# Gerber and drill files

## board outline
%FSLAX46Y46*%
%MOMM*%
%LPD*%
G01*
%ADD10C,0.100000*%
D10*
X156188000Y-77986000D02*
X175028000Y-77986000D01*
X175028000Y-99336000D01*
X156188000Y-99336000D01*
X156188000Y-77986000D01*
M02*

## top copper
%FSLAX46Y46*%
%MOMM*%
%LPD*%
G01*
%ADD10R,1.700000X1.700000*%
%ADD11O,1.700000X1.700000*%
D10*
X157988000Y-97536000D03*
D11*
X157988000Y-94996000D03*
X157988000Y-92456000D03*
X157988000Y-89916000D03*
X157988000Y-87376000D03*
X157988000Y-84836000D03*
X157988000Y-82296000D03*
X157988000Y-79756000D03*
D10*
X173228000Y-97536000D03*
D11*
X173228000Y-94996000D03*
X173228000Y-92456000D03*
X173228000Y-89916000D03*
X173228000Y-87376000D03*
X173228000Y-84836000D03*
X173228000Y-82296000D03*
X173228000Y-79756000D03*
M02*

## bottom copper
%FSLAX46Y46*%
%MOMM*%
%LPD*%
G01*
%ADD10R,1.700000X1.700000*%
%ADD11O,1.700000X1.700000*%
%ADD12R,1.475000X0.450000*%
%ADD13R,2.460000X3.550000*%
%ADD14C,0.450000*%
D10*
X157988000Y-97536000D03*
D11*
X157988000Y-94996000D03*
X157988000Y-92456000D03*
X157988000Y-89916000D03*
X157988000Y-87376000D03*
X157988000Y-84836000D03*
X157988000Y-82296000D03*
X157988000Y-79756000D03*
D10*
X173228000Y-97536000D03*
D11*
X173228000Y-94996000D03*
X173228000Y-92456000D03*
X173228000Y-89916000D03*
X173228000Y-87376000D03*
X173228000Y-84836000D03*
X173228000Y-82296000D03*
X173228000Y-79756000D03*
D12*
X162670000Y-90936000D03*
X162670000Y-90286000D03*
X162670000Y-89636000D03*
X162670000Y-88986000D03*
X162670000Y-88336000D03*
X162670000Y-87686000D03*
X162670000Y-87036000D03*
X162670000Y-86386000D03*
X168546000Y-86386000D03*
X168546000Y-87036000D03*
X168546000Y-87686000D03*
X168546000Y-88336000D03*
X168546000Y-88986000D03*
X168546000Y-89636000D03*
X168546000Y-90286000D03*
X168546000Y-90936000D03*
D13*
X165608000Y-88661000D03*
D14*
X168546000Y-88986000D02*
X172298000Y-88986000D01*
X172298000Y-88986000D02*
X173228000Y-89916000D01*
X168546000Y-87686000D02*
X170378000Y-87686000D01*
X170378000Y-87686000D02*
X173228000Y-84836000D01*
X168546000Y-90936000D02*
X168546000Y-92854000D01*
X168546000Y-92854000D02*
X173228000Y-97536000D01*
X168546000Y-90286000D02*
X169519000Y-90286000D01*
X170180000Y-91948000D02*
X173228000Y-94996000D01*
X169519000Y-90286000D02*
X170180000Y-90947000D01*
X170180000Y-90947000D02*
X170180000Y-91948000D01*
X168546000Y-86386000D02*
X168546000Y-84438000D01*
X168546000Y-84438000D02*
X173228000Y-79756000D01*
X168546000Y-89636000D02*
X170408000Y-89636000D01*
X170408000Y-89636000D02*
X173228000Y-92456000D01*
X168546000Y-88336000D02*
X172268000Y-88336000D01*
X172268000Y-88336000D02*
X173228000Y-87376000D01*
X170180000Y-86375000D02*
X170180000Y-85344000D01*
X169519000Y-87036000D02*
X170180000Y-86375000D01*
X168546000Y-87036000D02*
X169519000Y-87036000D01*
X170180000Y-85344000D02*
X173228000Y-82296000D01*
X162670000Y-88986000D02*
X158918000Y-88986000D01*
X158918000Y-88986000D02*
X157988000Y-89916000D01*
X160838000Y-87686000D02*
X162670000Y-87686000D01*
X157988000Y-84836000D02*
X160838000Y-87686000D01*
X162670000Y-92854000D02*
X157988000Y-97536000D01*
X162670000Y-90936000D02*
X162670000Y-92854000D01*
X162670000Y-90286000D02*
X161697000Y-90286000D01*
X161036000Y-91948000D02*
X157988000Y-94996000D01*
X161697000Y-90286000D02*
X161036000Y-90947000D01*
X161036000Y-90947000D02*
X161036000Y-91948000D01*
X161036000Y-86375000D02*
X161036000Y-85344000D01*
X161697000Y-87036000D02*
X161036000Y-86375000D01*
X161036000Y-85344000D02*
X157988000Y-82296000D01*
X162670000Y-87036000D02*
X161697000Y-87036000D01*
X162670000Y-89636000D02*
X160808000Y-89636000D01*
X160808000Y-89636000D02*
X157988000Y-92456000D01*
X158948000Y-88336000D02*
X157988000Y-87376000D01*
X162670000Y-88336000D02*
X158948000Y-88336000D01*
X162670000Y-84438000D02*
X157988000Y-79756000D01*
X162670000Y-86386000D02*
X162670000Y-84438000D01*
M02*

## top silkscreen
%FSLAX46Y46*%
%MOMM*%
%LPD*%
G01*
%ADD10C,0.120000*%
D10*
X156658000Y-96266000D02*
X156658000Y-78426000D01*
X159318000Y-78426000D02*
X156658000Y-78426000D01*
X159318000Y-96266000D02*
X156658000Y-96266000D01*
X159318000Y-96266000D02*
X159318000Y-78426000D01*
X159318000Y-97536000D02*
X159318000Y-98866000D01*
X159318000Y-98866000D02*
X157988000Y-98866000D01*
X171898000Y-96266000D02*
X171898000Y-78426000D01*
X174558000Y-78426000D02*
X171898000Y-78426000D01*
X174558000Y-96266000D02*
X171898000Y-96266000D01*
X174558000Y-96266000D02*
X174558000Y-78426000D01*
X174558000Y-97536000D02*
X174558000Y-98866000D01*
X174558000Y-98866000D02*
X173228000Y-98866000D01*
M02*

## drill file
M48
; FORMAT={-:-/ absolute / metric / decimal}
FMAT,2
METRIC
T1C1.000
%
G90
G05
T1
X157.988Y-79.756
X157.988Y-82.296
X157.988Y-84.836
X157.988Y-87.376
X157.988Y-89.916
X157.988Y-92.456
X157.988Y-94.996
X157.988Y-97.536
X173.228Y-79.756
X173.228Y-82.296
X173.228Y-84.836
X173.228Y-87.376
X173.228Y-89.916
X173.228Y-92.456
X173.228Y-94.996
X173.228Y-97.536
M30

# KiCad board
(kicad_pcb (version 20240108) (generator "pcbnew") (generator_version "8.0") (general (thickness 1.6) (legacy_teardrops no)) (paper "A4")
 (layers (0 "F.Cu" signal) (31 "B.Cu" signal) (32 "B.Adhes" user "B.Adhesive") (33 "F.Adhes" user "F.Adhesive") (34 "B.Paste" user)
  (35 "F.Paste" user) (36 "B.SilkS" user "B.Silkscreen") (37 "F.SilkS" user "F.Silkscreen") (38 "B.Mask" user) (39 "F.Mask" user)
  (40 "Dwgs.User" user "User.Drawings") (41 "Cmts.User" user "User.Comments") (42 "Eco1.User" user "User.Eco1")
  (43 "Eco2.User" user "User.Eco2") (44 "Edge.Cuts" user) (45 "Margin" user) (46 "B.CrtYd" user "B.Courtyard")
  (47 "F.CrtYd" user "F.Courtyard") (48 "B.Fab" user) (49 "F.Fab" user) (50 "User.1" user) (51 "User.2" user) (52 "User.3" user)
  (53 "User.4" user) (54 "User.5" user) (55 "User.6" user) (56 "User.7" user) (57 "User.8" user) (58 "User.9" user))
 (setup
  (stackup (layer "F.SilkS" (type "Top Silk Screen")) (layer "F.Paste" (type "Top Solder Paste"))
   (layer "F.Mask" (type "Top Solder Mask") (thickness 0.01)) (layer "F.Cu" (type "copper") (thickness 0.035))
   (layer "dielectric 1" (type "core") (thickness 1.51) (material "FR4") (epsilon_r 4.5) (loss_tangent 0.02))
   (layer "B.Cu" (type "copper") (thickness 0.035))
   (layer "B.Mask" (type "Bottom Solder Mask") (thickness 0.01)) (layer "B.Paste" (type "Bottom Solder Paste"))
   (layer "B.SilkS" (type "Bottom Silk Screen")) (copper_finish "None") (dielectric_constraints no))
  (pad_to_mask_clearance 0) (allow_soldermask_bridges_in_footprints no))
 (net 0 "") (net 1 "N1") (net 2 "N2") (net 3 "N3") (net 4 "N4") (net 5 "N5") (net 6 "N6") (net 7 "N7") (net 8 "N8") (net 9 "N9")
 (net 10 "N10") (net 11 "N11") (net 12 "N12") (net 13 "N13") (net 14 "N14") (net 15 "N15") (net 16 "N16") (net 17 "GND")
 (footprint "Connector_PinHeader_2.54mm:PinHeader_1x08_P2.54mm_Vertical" (layer "F.Cu") (at 157.988 97.536 180)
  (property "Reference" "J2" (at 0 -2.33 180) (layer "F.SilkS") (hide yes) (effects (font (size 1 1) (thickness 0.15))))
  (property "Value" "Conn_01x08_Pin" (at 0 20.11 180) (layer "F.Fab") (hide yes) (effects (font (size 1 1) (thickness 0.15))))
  (fp_line (start 1.33 1.27) (end 1.33 19.11) (stroke (width 0.12) (type solid)) (layer "F.SilkS"))
  (fp_line (start -1.33 19.11) (end 1.33 19.11) (stroke (width 0.12) (type solid)) (layer "F.SilkS"))
  (fp_line (start -1.33 1.27) (end 1.33 1.27) (stroke (width 0.12) (type solid)) (layer "F.SilkS"))
  (fp_line (start -1.33 1.27) (end -1.33 19.11) (stroke (width 0.12) (type solid)) (layer "F.SilkS"))
  (fp_line (start -1.33 0) (end -1.33 -1.33) (stroke (width 0.12) (type solid)) (layer "F.SilkS"))
  (fp_line (start -1.33 -1.33) (end 0 -1.33) (stroke (width 0.12) (type solid)) (layer "F.SilkS"))
  (pad "1" thru_hole rect (at 0 0 180) (size 1.7 1.7) (drill 1) (layers "*.Cu" "*.Mask") (remove_unused_layers no) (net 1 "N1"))
  (pad "2" thru_hole oval (at 0 2.54 180) (size 1.7 1.7) (drill 1) (layers "*.Cu" "*.Mask") (remove_unused_layers no) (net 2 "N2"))
  (pad "3" thru_hole oval (at 0 5.08 180) (size 1.7 1.7) (drill 1) (layers "*.Cu" "*.Mask") (remove_unused_layers no) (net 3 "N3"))
  (pad "4" thru_hole oval (at 0 7.62 180) (size 1.7 1.7) (drill 1) (layers "*.Cu" "*.Mask") (remove_unused_layers no) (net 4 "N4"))
  (pad "5" thru_hole oval (at 0 10.16 180) (size 1.7 1.7) (drill 1) (layers "*.Cu" "*.Mask") (remove_unused_layers no) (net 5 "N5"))
  (pad "6" thru_hole oval (at 0 12.7 180) (size 1.7 1.7) (drill 1) (layers "*.Cu" "*.Mask") (remove_unused_layers no) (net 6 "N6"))
  (pad "7" thru_hole oval (at 0 15.24 180) (size 1.7 1.7) (drill 1) (layers "*.Cu" "*.Mask") (remove_unused_layers no) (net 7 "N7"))
  (pad "8" thru_hole oval (at 0 17.78 180) (size 1.7 1.7) (drill 1) (layers "*.Cu" "*.Mask") (remove_unused_layers no) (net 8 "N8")))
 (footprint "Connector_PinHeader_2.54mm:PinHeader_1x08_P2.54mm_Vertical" (layer "F.Cu") (at 173.228 97.536 180)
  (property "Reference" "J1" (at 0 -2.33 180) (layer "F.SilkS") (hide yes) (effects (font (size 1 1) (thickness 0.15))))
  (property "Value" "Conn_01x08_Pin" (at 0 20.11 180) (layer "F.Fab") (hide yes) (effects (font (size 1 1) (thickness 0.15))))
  (fp_line (start 1.33 1.27) (end 1.33 19.11) (stroke (width 0.12) (type solid)) (layer "F.SilkS"))
  (fp_line (start -1.33 19.11) (end 1.33 19.11) (stroke (width 0.12) (type solid)) (layer "F.SilkS"))
  (fp_line (start -1.33 1.27) (end 1.33 1.27) (stroke (width 0.12) (type solid)) (layer "F.SilkS"))
  (fp_line (start -1.33 1.27) (end -1.33 19.11) (stroke (width 0.12) (type solid)) (layer "F.SilkS"))
  (fp_line (start -1.33 0) (end -1.33 -1.33) (stroke (width 0.12) (type solid)) (layer "F.SilkS"))
  (fp_line (start -1.33 -1.33) (end 0 -1.33) (stroke (width 0.12) (type solid)) (layer "F.SilkS"))
  (pad "1" thru_hole rect (at 0 0 180) (size 1.7 1.7) (drill 1) (layers "*.Cu" "*.Mask") (remove_unused_layers no) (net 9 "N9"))
  (pad "2" thru_hole oval (at 0 2.54 180) (size 1.7 1.7) (drill 1) (layers "*.Cu" "*.Mask") (remove_unused_layers no) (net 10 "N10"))
  (pad "3" thru_hole oval (at 0 5.08 180) (size 1.7 1.7) (drill 1) (layers "*.Cu" "*.Mask") (remove_unused_layers no) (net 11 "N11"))
  (pad "4" thru_hole oval (at 0 7.62 180) (size 1.7 1.7) (drill 1) (layers "*.Cu" "*.Mask") (remove_unused_layers no) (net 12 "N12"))
  (pad "5" thru_hole oval (at 0 10.16 180) (size 1.7 1.7) (drill 1) (layers "*.Cu" "*.Mask") (remove_unused_layers no) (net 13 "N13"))
  (pad "6" thru_hole oval (at 0 12.7 180) (size 1.7 1.7) (drill 1) (layers "*.Cu" "*.Mask") (remove_unused_layers no) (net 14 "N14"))
  (pad "7" thru_hole oval (at 0 15.24 180) (size 1.7 1.7) (drill 1) (layers "*.Cu" "*.Mask") (remove_unused_layers no) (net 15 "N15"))
  (pad "8" thru_hole oval (at 0 17.78 180) (size 1.7 1.7) (drill 1) (layers "*.Cu" "*.Mask") (remove_unused_layers no) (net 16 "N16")))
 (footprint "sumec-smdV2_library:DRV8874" (layer "B.Cu") (at 165.608 88.661)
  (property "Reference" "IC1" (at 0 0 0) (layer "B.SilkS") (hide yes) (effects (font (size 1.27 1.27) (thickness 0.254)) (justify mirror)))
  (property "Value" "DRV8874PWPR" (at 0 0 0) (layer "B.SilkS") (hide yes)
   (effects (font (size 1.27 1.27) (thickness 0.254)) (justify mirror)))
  (pad "1" smd rect (at -2.938 2.275 270) (size 0.45 1.475) (layers "B.Cu" "B.Paste" "B.Mask") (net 1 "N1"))
  (pad "2" smd rect (at -2.938 1.625 270) (size 0.45 1.475) (layers "B.Cu" "B.Paste" "B.Mask") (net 2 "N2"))
  (pad "3" smd rect (at -2.938 0.975 270) (size 0.45 1.475) (layers "B.Cu" "B.Paste" "B.Mask") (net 3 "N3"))
  (pad "4" smd rect (at -2.938 0.325 270) (size 0.45 1.475) (layers "B.Cu" "B.Paste" "B.Mask") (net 4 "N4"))
  (pad "5" smd rect (at -2.938 -0.325 270) (size 0.45 1.475) (layers "B.Cu" "B.Paste" "B.Mask") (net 5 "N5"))
  (pad "6" smd rect (at -2.938 -0.975 270) (size 0.45 1.475) (layers "B.Cu" "B.Paste" "B.Mask") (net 6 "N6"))
  (pad "7" smd rect (at -2.938 -1.625 270) (size 0.45 1.475) (layers "B.Cu" "B.Paste" "B.Mask") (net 7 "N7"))
  (pad "8" smd rect (at -2.938 -2.275 270) (size 0.45 1.475) (layers "B.Cu" "B.Paste" "B.Mask") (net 8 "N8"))
  (pad "9" smd rect (at 2.938 -2.275 270) (size 0.45 1.475) (layers "B.Cu" "B.Paste" "B.Mask") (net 16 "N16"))
  (pad "10" smd rect (at 2.938 -1.625 270) (size 0.45 1.475) (layers "B.Cu" "B.Paste" "B.Mask") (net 15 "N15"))
  (pad "11" smd rect (at 2.938 -0.975 270) (size 0.45 1.475) (layers "B.Cu" "B.Paste" "B.Mask") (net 14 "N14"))
  (pad "12" smd rect (at 2.938 -0.325 270) (size 0.45 1.475) (layers "B.Cu" "B.Paste" "B.Mask") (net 13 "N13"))
  (pad "13" smd rect (at 2.938 0.325 270) (size 0.45 1.475) (layers "B.Cu" "B.Paste" "B.Mask") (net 12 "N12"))
  (pad "14" smd rect (at 2.938 0.975 270) (size 0.45 1.475) (layers "B.Cu" "B.Paste" "B.Mask") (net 11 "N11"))
  (pad "15" smd rect (at 2.938 1.625 270) (size 0.45 1.475) (layers "B.Cu" "B.Paste" "B.Mask") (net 10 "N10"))
  (pad "16" smd rect (at 2.938 2.275 270) (size 0.45 1.475) (layers "B.Cu" "B.Paste" "B.Mask") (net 9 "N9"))
  (pad "17" smd rect (at 0 0) (size 2.46 3.55) (layers "B.Cu" "B.Paste" "B.Mask") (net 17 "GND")))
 (gr_rect (start 156.188 77.986) (end 175.028 99.336) (stroke (width 0.1) (type default)) (fill none) (layer "Edge.Cuts"))
 (segment (start 168.546 88.986) (end 172.298 88.986) (width 0.45) (layer "B.Cu") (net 12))
 (segment (start 172.298 88.986) (end 173.228 89.916) (width 0.45) (layer "B.Cu") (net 12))
 (segment (start 168.546 87.686) (end 170.378 87.686) (width 0.45) (layer "B.Cu") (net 14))
 (segment (start 170.378 87.686) (end 173.228 84.836) (width 0.45) (layer "B.Cu") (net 14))
 (segment (start 168.546 90.936) (end 168.546 92.854) (width 0.45) (layer "B.Cu") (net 9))
 (segment (start 168.546 92.854) (end 173.228 97.536) (width 0.45) (layer "B.Cu") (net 9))
 (segment (start 168.546 90.286) (end 169.519 90.286) (width 0.45) (layer "B.Cu") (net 10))
 (segment (start 170.18 91.948) (end 173.228 94.996) (width 0.45) (layer "B.Cu") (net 10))
 (segment (start 169.519 90.286) (end 170.18 90.947) (width 0.45) (layer "B.Cu") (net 10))
 (segment (start 170.18 90.947) (end 170.18 91.948) (width 0.45) (layer "B.Cu") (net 10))
 (segment (start 168.546 86.386) (end 168.546 84.438) (width 0.45) (layer "B.Cu") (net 16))
 (segment (start 168.546 84.438) (end 173.228 79.756) (width 0.45) (layer "B.Cu") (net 16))
 (segment (start 168.546 89.636) (end 170.408 89.636) (width 0.45) (layer "B.Cu") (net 11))
 (segment (start 170.408 89.636) (end 173.228 92.456) (width 0.45) (layer "B.Cu") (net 11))
 (segment (start 168.546 88.336) (end 172.268 88.336) (width 0.45) (layer "B.Cu") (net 13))
 (segment (start 172.268 88.336) (end 173.228 87.376) (width 0.45) (layer "B.Cu") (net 13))
 (segment (start 170.18 86.375) (end 170.18 85.344) (width 0.45) (layer "B.Cu") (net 15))
 (segment (start 169.519 87.036) (end 170.18 86.375) (width 0.45) (layer "B.Cu") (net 15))
 (segment (start 168.546 87.036) (end 169.519 87.036) (width 0.45) (layer "B.Cu") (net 15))
 (segment (start 170.18 85.344) (end 173.228 82.296) (width 0.45) (layer "B.Cu") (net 15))
 (segment (start 162.67 88.986) (end 158.918 88.986) (width 0.45) (layer "B.Cu") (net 4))
 (segment (start 158.918 88.986) (end 157.988 89.916) (width 0.45) (layer "B.Cu") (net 4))
 (segment (start 160.838 87.686) (end 162.67 87.686) (width 0.45) (layer "B.Cu") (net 6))
 (segment (start 157.988 84.836) (end 160.838 87.686) (width 0.45) (layer "B.Cu") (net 6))
 (segment (start 162.67 92.854) (end 157.988 97.536) (width 0.45) (layer "B.Cu") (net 1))
 (segment (start 162.67 90.936) (end 162.67 92.854) (width 0.45) (layer "B.Cu") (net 1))
 (segment (start 162.67 90.286) (end 161.697 90.286) (width 0.45) (layer "B.Cu") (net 2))
 (segment (start 161.036 91.948) (end 157.988 94.996) (width 0.45) (layer "B.Cu") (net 2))
 (segment (start 161.697 90.286) (end 161.036 90.947) (width 0.45) (layer "B.Cu") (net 2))
 (segment (start 161.036 90.947) (end 161.036 91.948) (width 0.45) (layer "B.Cu") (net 2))
 (segment (start 161.036 86.375) (end 161.036 85.344) (width 0.45) (layer "B.Cu") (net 7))
 (segment (start 161.697 87.036) (end 161.036 86.375) (width 0.45) (layer "B.Cu") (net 7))
 (segment (start 161.036 85.344) (end 157.988 82.296) (width 0.45) (layer "B.Cu") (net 7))
 (segment (start 162.67 87.036) (end 161.697 87.036) (width 0.45) (layer "B.Cu") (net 7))
 (segment (start 162.67 89.636) (end 160.808 89.636) (width 0.45) (layer "B.Cu") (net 3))
 (segment (start 160.808 89.636) (end 157.988 92.456) (width 0.45) (layer "B.Cu") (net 3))
 (segment (start 158.948 88.336) (end 157.988 87.376) (width 0.45) (layer "B.Cu") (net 5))
 (segment (start 162.67 88.336) (end 158.948 88.336) (width 0.45) (layer "B.Cu") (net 5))
 (segment (start 162.67 84.438) (end 157.988 79.756) (width 0.45) (layer "B.Cu") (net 8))
 (segment (start 162.67 86.386) (end 162.67 84.438) (width 0.45) (layer "B.Cu") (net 8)))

